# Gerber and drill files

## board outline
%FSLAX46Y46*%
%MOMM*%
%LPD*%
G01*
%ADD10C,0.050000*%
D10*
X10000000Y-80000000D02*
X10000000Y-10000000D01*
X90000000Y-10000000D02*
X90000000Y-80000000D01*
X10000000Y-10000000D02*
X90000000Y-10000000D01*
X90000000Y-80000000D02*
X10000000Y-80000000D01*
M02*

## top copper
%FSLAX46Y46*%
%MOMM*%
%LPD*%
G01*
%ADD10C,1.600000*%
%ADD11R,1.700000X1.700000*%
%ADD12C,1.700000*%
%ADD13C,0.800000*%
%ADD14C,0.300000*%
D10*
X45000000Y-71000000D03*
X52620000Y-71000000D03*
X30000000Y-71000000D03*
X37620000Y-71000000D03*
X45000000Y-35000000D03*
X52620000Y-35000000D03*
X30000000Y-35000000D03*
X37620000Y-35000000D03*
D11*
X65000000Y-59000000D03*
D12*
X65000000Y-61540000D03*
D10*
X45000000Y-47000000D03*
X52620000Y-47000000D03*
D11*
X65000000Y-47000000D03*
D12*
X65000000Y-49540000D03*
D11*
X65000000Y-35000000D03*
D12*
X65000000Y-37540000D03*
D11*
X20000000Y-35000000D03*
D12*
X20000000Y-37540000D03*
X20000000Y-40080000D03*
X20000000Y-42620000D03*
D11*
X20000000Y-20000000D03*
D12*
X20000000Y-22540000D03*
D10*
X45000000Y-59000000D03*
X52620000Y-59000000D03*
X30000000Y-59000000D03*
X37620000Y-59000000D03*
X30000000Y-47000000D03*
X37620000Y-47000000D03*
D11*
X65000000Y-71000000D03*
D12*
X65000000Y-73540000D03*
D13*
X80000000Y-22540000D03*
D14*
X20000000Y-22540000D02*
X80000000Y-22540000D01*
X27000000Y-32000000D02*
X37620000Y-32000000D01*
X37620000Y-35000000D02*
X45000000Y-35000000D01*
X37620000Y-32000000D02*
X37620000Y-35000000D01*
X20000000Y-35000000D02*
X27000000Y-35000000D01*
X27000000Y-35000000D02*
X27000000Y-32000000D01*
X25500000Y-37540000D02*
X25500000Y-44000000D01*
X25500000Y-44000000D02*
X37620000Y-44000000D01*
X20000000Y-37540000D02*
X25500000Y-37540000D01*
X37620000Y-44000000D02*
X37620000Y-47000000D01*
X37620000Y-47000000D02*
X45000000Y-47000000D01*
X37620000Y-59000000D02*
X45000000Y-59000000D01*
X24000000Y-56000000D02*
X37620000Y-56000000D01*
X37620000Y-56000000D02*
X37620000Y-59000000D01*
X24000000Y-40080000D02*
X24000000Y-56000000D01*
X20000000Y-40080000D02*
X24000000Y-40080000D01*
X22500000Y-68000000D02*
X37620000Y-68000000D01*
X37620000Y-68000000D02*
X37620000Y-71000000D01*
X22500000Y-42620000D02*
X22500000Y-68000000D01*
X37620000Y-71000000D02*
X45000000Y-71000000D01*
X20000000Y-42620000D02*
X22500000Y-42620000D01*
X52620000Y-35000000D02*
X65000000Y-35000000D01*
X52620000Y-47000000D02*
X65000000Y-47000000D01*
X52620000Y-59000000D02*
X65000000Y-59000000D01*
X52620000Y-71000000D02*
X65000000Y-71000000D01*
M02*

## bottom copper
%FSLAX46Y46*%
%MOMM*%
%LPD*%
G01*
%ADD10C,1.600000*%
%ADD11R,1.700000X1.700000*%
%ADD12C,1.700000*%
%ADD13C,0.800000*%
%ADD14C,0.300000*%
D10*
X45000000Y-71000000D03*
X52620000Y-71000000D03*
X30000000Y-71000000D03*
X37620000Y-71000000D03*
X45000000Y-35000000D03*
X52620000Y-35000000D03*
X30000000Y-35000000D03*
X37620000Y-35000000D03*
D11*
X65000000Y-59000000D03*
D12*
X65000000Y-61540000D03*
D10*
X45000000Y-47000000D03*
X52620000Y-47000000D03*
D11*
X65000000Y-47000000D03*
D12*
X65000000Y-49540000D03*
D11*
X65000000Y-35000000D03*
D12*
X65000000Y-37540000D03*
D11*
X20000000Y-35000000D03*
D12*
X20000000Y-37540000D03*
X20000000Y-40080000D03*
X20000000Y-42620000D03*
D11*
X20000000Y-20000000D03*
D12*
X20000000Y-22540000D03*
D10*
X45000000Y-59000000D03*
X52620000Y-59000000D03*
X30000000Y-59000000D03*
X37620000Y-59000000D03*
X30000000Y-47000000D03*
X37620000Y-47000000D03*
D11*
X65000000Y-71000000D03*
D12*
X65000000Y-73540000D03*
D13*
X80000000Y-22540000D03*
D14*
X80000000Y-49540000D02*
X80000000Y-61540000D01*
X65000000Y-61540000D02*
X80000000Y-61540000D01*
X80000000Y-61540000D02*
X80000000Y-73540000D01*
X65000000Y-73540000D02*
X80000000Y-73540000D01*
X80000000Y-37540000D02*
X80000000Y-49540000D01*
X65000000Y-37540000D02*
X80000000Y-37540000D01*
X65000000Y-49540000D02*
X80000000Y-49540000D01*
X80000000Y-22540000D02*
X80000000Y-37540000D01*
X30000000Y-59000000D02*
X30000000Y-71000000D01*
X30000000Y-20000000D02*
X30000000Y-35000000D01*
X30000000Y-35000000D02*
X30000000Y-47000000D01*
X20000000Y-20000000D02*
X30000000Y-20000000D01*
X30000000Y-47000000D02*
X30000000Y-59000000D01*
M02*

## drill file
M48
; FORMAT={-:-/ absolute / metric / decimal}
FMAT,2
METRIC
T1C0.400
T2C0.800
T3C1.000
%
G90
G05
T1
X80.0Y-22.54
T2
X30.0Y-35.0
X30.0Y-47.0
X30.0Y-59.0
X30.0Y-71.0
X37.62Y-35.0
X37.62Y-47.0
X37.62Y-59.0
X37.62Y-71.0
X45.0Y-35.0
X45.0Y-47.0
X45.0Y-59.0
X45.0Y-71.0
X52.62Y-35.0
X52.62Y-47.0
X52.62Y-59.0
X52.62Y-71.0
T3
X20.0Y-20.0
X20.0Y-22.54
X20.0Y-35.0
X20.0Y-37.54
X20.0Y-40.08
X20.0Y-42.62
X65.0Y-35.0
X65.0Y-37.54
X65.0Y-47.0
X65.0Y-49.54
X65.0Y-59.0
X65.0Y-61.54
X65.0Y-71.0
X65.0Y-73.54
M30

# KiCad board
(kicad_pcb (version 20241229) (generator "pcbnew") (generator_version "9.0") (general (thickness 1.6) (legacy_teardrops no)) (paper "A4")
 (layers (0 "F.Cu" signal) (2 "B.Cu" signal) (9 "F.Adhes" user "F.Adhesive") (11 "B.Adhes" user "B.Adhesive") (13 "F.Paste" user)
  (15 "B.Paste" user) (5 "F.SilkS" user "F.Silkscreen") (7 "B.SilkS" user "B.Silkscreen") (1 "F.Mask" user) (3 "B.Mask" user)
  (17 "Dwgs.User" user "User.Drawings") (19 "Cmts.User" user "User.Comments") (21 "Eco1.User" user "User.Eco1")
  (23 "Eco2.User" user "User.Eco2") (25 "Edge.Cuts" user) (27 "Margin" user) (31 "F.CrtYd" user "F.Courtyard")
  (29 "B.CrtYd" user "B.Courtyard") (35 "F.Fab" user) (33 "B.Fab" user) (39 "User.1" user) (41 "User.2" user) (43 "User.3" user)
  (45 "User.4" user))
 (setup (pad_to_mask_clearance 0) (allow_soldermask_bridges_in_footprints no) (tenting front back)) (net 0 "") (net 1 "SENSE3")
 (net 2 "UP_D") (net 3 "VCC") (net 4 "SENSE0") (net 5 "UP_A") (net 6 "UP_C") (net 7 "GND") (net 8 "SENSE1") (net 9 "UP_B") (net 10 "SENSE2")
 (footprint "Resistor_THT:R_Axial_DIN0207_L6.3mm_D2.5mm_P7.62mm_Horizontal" (layer "F.Cu") (at 45 71)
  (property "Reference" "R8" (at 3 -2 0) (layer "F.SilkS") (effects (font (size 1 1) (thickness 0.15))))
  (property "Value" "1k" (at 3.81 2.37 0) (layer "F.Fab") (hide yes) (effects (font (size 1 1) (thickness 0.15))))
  (pad "1" thru_hole circle (at 0 0) (size 1.6 1.6) (drill 0.8) (layers "*.Cu" "*.Mask") (remove_unused_layers no) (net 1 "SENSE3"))
  (pad "2" thru_hole circle (at 7.62 0) (size 1.6 1.6) (drill 0.8) (layers "*.Cu" "*.Mask") (remove_unused_layers no) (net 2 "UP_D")))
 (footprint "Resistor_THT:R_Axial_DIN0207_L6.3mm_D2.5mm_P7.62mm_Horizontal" (layer "F.Cu") (at 30 71)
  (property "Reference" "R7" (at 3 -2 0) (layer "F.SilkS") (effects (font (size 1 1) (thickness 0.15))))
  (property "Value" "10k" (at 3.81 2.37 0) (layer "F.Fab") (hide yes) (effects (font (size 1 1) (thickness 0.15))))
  (pad "1" thru_hole circle (at 0 0) (size 1.6 1.6) (drill 0.8) (layers "*.Cu" "*.Mask") (remove_unused_layers no) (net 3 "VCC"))
  (pad "2" thru_hole circle (at 7.62 0) (size 1.6 1.6) (drill 0.8) (layers "*.Cu" "*.Mask") (remove_unused_layers no) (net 1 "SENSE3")))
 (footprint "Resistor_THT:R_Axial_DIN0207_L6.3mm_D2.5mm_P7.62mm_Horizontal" (layer "F.Cu") (at 45 35)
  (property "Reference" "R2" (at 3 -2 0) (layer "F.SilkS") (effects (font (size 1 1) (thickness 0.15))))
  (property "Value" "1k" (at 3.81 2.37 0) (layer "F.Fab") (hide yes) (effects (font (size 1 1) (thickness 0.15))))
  (pad "1" thru_hole circle (at 0 0) (size 1.6 1.6) (drill 0.8) (layers "*.Cu" "*.Mask") (remove_unused_layers no) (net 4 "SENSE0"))
  (pad "2" thru_hole circle (at 7.62 0) (size 1.6 1.6) (drill 0.8) (layers "*.Cu" "*.Mask") (remove_unused_layers no) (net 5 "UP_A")))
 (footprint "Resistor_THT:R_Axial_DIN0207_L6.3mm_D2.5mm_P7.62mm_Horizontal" (layer "F.Cu") (at 30 35)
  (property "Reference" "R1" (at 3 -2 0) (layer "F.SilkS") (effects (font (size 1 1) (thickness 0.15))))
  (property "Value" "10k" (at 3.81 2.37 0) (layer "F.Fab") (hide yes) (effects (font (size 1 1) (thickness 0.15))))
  (pad "1" thru_hole circle (at 0 0) (size 1.6 1.6) (drill 0.8) (layers "*.Cu" "*.Mask") (remove_unused_layers no) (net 3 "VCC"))
  (pad "2" thru_hole circle (at 7.62 0) (size 1.6 1.6) (drill 0.8) (layers "*.Cu" "*.Mask") (remove_unused_layers no) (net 4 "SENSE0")))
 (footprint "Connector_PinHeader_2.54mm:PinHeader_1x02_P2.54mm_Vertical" (layer "F.Cu") (at 65 59)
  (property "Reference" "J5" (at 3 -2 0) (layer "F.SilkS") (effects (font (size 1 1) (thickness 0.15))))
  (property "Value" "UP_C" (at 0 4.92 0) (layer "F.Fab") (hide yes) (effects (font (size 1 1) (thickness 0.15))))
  (pad "1" thru_hole rect (at 0 0) (size 1.7 1.7) (drill 1) (layers "*.Cu" "*.Mask") (remove_unused_layers no) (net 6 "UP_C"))
  (pad "2" thru_hole circle (at 0 2.54) (size 1.7 1.7) (drill 1) (layers "*.Cu" "*.Mask") (remove_unused_layers no) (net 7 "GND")))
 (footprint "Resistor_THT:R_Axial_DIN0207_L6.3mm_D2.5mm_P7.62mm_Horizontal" (layer "F.Cu") (at 45 47)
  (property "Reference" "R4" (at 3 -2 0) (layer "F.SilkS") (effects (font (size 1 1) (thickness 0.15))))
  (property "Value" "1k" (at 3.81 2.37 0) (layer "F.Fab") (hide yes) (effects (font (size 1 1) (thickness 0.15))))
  (pad "1" thru_hole circle (at 0 0) (size 1.6 1.6) (drill 0.8) (layers "*.Cu" "*.Mask") (remove_unused_layers no) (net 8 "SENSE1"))
  (pad "2" thru_hole circle (at 7.62 0) (size 1.6 1.6) (drill 0.8) (layers "*.Cu" "*.Mask") (remove_unused_layers no) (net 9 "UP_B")))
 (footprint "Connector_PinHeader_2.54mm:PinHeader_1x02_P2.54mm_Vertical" (layer "F.Cu") (at 65 47)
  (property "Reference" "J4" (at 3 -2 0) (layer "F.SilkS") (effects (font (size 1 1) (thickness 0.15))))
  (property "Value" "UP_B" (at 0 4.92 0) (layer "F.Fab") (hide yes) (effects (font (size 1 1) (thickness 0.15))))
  (pad "1" thru_hole rect (at 0 0) (size 1.7 1.7) (drill 1) (layers "*.Cu" "*.Mask") (remove_unused_layers no) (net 9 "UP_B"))
  (pad "2" thru_hole circle (at 0 2.54) (size 1.7 1.7) (drill 1) (layers "*.Cu" "*.Mask") (remove_unused_layers no) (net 7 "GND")))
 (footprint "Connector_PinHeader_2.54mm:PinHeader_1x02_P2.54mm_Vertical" (layer "F.Cu") (at 65 35)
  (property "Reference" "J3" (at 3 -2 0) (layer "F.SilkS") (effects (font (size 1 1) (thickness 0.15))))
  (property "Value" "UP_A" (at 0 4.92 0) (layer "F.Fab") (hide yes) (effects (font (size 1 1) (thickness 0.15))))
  (pad "1" thru_hole rect (at 0 0) (size 1.7 1.7) (drill 1) (layers "*.Cu" "*.Mask") (remove_unused_layers no) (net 5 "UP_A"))
  (pad "2" thru_hole circle (at 0 2.54) (size 1.7 1.7) (drill 1) (layers "*.Cu" "*.Mask") (remove_unused_layers no) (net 7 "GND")))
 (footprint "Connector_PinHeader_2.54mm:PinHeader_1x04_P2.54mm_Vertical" (layer "F.Cu") (at 20 35)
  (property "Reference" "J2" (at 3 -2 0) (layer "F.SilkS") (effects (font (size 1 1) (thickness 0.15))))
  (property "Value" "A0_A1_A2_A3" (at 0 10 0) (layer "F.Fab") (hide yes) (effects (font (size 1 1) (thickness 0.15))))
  (pad "1" thru_hole rect (at 0 0) (size 1.7 1.7) (drill 1) (layers "*.Cu" "*.Mask") (remove_unused_layers no) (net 4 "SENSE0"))
  (pad "2" thru_hole circle (at 0 2.54) (size 1.7 1.7) (drill 1) (layers "*.Cu" "*.Mask") (remove_unused_layers no) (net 8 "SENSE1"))
  (pad "3" thru_hole circle (at 0 5.08) (size 1.7 1.7) (drill 1) (layers "*.Cu" "*.Mask") (remove_unused_layers no) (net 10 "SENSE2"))
  (pad "4" thru_hole circle (at 0 7.62) (size 1.7 1.7) (drill 1) (layers "*.Cu" "*.Mask") (remove_unused_layers no) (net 1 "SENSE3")))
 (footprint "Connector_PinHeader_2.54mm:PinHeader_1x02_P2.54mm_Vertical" (layer "F.Cu") (at 20 20)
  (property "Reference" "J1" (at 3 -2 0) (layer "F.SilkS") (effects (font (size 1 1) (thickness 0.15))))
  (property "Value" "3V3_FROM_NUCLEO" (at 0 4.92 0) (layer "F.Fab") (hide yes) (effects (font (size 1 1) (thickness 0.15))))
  (pad "1" thru_hole rect (at 0 0) (size 1.7 1.7) (drill 1) (layers "*.Cu" "*.Mask") (remove_unused_layers no) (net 3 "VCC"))
  (pad "2" thru_hole circle (at 0 2.54) (size 1.7 1.7) (drill 1) (layers "*.Cu" "*.Mask") (remove_unused_layers no) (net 7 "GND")))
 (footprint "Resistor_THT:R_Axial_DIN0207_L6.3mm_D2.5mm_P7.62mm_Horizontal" (layer "F.Cu") (at 45 59)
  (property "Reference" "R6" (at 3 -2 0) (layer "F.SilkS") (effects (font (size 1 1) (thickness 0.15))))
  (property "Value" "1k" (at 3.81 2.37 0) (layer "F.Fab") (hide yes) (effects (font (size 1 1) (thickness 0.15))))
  (pad "1" thru_hole circle (at 0 0) (size 1.6 1.6) (drill 0.8) (layers "*.Cu" "*.Mask") (remove_unused_layers no) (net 10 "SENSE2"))
  (pad "2" thru_hole circle (at 7.62 0) (size 1.6 1.6) (drill 0.8) (layers "*.Cu" "*.Mask") (remove_unused_layers no) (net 6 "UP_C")))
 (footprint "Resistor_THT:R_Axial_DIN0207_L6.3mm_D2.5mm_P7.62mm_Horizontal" (layer "F.Cu") (at 30 59)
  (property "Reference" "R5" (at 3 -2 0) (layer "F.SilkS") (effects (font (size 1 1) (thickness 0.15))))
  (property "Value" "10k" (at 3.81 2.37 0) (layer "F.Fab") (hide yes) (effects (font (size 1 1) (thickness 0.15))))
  (pad "1" thru_hole circle (at 0 0) (size 1.6 1.6) (drill 0.8) (layers "*.Cu" "*.Mask") (remove_unused_layers no) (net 3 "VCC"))
  (pad "2" thru_hole circle (at 7.62 0) (size 1.6 1.6) (drill 0.8) (layers "*.Cu" "*.Mask") (remove_unused_layers no) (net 10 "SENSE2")))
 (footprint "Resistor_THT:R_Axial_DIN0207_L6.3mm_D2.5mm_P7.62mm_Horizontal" (layer "F.Cu") (at 30 47)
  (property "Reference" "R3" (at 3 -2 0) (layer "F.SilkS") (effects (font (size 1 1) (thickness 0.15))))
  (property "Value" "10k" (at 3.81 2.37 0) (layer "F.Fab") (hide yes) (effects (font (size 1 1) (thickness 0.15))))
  (pad "1" thru_hole circle (at 0 0) (size 1.6 1.6) (drill 0.8) (layers "*.Cu" "*.Mask") (remove_unused_layers no) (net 3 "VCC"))
  (pad "2" thru_hole circle (at 7.62 0) (size 1.6 1.6) (drill 0.8) (layers "*.Cu" "*.Mask") (remove_unused_layers no) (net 8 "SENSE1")))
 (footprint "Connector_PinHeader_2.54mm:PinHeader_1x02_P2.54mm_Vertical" (layer "F.Cu") (at 65 71)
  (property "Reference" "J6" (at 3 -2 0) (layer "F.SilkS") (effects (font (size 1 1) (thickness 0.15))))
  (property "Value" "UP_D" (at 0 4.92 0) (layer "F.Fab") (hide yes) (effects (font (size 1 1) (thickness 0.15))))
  (pad "1" thru_hole rect (at 0 0) (size 1.7 1.7) (drill 1) (layers "*.Cu" "*.Mask") (remove_unused_layers no) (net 2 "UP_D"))
  (pad "2" thru_hole circle (at 0 2.54) (size 1.7 1.7) (drill 1) (layers "*.Cu" "*.Mask") (remove_unused_layers no) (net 7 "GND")))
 (gr_line (start 10 80) (end 10 10) (stroke (width 0.05) (type default)) (layer "Edge.Cuts"))
 (gr_line (start 90 10) (end 90 80) (stroke (width 0.05) (type default)) (layer "Edge.Cuts"))
 (gr_line (start 10 10) (end 90 10) (stroke (width 0.05) (type default)) (layer "Edge.Cuts"))
 (gr_line (start 90 80) (end 10 80) (stroke (width 0.05) (type default)) (layer "Edge.Cuts"))
 (segment (start 20 22.54) (end 80 22.54) (width 0.3) (layer "F.Cu") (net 7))
 (via (at 80 22.54) (size 0.8) (drill 0.4) (layers "F.Cu" "B.Cu") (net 7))
 (segment (start 80 49.54) (end 80 61.54) (width 0.3) (layer "B.Cu") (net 7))
 (segment (start 65 61.54) (end 80 61.54) (width 0.3) (layer "B.Cu") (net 7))
 (segment (start 80 61.54) (end 80 73.54) (width 0.3) (layer "B.Cu") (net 7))
 (segment (start 65 73.54) (end 80 73.54) (width 0.3) (layer "B.Cu") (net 7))
 (segment (start 80 37.54) (end 80 49.54) (width 0.3) (layer "B.Cu") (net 7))
 (segment (start 65 37.54) (end 80 37.54) (width 0.3) (layer "B.Cu") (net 7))
 (segment (start 65 49.54) (end 80 49.54) (width 0.3) (layer "B.Cu") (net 7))
 (segment (start 80 22.54) (end 80 37.54) (width 0.3) (layer "B.Cu") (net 7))
 (segment (start 27 32) (end 37.62 32) (width 0.3) (layer "F.Cu") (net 4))
 (segment (start 37.62 35) (end 45 35) (width 0.3) (layer "F.Cu") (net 4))
 (segment (start 37.62 32) (end 37.62 35) (width 0.3) (layer "F.Cu") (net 4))
 (segment (start 20 35) (end 27 35) (width 0.3) (layer "F.Cu") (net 4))
 (segment (start 27 35) (end 27 32) (width 0.3) (layer "F.Cu") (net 4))
 (segment (start 25.5 37.54) (end 25.5 44) (width 0.3) (layer "F.Cu") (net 8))
 (segment (start 25.5 44) (end 37.62 44) (width 0.3) (layer "F.Cu") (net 8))
 (segment (start 20 37.54) (end 25.5 37.54) (width 0.3) (layer "F.Cu") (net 8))
 (segment (start 37.62 44) (end 37.62 47) (width 0.3) (layer "F.Cu") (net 8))
 (segment (start 37.62 47) (end 45 47) (width 0.3) (layer "F.Cu") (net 8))
 (segment (start 37.62 59) (end 45 59) (width 0.3) (layer "F.Cu") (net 10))
 (segment (start 24 56) (end 37.62 56) (width 0.3) (layer "F.Cu") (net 10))
 (segment (start 37.62 56) (end 37.62 59) (width 0.3) (layer "F.Cu") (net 10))
 (segment (start 24 40.08) (end 24 56) (width 0.3) (layer "F.Cu") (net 10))
 (segment (start 20 40.08) (end 24 40.08) (width 0.3) (layer "F.Cu") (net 10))
 (segment (start 22.5 68) (end 37.62 68) (width 0.3) (layer "F.Cu") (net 1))
 (segment (start 37.62 68) (end 37.62 71) (width 0.3) (layer "F.Cu") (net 1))
 (segment (start 22.5 42.62) (end 22.5 68) (width 0.3) (layer "F.Cu") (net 1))
 (segment (start 37.62 71) (end 45 71) (width 0.3) (layer "F.Cu") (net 1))
 (segment (start 20 42.62) (end 22.5 42.62) (width 0.3) (layer "F.Cu") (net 1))
 (segment (start 52.62 35) (end 65 35) (width 0.3) (layer "F.Cu") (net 5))
 (segment (start 52.62 47) (end 65 47) (width 0.3) (layer "F.Cu") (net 9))
 (segment (start 52.62 59) (end 65 59) (width 0.3) (layer "F.Cu") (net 6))
 (segment (start 52.62 71) (end 65 71) (width 0.3) (layer "F.Cu") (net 2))
 (segment (start 30 59) (end 30 71) (width 0.3) (layer "B.Cu") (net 3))
 (segment (start 30 20) (end 30 35) (width 0.3) (layer "B.Cu") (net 3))
 (segment (start 30 35) (end 30 47) (width 0.3) (layer "B.Cu") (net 3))
 (segment (start 20 20) (end 30 20) (width 0.3) (layer "B.Cu") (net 3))
 (segment (start 30 47) (end 30 59) (width 0.3) (layer "B.Cu") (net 3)))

